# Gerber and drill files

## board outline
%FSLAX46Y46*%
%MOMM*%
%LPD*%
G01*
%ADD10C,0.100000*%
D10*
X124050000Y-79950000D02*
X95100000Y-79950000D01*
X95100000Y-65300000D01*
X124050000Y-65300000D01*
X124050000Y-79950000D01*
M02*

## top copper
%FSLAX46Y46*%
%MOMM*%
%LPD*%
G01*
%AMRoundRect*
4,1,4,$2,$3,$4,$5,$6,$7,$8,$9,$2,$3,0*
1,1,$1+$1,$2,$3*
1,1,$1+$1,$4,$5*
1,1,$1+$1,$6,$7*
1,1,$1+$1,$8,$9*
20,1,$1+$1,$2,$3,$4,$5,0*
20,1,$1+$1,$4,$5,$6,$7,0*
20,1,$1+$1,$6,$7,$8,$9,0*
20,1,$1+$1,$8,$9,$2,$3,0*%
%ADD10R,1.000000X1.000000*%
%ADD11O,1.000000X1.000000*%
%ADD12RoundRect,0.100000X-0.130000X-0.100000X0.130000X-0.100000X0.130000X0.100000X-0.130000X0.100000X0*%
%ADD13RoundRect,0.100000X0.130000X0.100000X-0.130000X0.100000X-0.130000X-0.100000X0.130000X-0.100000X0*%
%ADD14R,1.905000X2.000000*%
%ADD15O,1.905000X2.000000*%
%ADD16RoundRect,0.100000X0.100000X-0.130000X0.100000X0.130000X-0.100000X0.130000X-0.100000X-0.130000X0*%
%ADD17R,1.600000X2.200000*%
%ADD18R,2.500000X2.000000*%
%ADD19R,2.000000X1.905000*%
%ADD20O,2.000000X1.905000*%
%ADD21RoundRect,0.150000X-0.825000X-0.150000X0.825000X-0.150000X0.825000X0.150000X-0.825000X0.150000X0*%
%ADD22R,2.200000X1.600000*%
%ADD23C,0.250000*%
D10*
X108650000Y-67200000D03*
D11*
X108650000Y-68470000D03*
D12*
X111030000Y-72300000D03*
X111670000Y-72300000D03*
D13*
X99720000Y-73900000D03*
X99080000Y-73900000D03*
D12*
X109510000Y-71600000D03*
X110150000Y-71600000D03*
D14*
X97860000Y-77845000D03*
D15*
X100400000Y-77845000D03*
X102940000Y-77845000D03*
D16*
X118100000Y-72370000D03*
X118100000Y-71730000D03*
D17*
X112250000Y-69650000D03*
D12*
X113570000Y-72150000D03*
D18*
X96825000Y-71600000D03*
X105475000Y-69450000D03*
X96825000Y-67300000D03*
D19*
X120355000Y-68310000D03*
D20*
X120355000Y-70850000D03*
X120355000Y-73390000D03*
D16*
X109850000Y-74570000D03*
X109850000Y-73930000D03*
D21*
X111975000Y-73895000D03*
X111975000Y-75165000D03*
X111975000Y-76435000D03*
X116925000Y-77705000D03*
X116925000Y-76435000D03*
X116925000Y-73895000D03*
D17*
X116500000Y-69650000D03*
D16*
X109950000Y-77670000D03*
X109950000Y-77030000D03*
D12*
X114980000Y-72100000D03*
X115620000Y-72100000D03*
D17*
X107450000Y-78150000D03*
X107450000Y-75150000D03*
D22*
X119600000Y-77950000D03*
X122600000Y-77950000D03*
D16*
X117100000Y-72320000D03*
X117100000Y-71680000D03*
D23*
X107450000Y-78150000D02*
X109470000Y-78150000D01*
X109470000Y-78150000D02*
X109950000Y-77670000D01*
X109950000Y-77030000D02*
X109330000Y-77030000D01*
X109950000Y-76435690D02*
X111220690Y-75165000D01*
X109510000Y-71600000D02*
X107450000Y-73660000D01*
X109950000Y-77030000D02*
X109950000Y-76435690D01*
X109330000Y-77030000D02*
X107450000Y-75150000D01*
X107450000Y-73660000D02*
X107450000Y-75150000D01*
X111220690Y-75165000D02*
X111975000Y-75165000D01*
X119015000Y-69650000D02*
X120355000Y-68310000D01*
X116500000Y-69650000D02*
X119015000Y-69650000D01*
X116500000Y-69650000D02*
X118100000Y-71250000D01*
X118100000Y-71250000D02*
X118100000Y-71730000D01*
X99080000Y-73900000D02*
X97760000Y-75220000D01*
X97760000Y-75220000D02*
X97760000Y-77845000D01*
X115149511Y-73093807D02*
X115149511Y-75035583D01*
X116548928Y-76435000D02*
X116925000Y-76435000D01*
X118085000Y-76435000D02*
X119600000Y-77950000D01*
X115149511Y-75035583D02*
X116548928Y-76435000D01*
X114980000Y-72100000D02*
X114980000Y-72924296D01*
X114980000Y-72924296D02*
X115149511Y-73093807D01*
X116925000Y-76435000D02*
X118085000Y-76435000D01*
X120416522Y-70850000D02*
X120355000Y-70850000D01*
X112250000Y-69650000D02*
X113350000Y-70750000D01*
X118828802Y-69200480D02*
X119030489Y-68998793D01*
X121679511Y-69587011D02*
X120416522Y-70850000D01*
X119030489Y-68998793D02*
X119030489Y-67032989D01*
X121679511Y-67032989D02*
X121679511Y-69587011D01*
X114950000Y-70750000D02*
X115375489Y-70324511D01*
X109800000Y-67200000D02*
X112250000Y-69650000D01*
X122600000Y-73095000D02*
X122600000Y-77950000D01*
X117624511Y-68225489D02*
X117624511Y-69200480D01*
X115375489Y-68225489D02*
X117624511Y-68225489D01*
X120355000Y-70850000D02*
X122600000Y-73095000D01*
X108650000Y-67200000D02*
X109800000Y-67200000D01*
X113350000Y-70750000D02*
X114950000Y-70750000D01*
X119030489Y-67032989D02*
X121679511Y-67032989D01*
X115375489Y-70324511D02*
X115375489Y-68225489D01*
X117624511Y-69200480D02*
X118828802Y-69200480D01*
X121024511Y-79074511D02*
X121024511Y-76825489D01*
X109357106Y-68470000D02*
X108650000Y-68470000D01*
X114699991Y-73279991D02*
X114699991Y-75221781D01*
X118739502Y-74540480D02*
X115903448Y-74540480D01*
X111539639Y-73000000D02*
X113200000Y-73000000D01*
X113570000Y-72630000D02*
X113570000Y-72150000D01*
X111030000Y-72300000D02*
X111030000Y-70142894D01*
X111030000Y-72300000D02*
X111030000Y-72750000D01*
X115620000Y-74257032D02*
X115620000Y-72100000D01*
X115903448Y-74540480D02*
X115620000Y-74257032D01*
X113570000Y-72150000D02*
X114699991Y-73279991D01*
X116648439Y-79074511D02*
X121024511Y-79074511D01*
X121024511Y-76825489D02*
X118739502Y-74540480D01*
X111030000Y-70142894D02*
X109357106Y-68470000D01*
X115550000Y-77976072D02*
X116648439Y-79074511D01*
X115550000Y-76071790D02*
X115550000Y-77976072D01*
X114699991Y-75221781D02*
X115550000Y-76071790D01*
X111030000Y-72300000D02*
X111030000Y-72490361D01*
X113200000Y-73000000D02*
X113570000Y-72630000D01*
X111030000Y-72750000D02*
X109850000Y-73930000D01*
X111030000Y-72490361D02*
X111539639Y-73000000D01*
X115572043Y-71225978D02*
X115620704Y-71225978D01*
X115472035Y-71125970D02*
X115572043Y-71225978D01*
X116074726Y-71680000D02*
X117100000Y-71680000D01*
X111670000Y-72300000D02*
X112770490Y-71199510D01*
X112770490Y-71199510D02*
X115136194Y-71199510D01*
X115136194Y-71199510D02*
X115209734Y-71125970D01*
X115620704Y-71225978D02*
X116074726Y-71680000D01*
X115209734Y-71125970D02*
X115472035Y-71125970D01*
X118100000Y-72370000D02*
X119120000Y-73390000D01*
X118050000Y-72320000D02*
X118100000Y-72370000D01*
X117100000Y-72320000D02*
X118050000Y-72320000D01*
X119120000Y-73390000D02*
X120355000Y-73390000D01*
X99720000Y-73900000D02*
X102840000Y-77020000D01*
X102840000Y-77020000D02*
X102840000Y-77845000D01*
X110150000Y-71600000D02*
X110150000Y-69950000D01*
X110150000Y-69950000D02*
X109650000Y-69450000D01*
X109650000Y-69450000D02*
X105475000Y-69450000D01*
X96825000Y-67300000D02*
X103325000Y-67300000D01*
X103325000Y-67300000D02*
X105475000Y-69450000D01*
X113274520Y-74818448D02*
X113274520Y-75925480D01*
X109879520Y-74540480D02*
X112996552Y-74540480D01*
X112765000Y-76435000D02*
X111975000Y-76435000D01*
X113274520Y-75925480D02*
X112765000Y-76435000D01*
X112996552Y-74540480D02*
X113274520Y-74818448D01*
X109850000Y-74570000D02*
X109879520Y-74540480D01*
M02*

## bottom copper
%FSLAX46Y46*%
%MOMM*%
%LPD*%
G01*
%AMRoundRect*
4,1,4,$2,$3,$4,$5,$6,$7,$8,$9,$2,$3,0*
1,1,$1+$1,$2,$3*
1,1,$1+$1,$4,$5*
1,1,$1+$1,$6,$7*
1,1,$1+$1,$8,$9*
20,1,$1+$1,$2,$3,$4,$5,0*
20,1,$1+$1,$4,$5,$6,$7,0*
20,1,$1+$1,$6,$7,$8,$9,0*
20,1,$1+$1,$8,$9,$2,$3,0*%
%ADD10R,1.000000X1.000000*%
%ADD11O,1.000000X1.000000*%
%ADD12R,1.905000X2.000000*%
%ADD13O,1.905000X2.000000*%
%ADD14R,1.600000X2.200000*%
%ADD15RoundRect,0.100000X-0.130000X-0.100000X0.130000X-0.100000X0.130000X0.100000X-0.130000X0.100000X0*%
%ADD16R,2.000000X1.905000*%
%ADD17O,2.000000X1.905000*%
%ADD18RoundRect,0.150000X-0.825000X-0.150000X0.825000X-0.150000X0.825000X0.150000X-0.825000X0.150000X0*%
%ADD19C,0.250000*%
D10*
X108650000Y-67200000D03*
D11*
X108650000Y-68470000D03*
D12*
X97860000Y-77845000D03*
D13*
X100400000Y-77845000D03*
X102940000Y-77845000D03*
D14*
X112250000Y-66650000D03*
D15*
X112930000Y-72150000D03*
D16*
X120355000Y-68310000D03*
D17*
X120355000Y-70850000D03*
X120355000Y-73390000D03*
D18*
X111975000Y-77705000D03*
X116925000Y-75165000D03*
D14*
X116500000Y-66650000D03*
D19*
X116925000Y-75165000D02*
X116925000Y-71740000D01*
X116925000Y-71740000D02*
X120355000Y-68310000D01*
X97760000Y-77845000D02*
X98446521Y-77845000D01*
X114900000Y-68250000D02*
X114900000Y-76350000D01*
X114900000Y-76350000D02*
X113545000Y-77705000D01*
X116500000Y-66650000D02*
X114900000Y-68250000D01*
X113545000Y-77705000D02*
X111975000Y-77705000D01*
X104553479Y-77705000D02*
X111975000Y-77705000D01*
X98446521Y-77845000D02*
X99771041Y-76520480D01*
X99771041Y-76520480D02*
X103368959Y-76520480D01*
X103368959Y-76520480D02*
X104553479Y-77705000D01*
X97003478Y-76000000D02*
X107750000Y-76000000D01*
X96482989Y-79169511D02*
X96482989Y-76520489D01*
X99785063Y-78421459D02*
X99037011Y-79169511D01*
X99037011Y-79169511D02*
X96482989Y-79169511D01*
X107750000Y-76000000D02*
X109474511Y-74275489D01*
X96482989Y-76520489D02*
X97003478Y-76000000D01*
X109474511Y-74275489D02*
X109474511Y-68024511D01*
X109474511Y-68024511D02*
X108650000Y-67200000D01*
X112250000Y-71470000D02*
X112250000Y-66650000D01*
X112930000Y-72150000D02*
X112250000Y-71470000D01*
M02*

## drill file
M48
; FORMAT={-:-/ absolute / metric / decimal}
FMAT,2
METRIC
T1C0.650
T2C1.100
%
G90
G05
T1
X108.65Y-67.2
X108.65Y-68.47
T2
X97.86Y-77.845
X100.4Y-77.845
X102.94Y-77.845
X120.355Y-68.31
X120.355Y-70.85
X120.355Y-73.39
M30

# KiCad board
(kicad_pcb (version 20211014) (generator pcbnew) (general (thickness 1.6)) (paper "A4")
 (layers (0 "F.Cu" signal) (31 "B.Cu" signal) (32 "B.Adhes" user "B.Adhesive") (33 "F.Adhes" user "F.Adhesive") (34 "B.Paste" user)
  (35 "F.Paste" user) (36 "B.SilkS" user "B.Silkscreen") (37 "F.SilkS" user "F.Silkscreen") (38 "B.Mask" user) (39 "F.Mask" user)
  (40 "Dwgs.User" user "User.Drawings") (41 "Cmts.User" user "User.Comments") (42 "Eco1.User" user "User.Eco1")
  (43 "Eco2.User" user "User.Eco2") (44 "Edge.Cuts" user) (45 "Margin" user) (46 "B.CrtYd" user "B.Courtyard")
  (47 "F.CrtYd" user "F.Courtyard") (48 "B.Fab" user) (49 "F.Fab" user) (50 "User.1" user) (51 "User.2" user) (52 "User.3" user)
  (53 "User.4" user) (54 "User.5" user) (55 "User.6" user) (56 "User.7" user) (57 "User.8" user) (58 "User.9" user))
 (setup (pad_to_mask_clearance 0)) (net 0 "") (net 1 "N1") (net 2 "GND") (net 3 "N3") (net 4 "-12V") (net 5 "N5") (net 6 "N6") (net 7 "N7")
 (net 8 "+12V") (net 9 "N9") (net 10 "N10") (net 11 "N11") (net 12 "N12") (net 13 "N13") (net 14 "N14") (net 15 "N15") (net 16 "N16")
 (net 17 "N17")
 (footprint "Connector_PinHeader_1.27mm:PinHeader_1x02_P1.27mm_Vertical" (layer "F.Cu") (at 108.65 67.2)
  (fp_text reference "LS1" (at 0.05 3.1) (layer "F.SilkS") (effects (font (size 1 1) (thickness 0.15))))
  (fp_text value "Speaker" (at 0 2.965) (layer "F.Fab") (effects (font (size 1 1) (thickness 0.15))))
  (pad "1" thru_hole rect (at 0 0) (size 1 1) (drill 0.65) (layers *.Cu *.Mask) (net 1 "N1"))
  (pad "2" thru_hole oval (at 0 1.27) (size 1 1) (drill 0.65) (layers *.Cu *.Mask) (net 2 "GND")))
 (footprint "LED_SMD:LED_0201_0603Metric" (layer "F.Cu") (at 111.35 72.3)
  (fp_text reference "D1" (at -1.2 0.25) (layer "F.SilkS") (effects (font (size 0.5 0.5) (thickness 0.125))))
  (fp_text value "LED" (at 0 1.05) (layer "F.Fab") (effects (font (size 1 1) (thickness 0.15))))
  (pad "" smd roundrect (at 0.345 0) (size 0.318 0.36) (layers "F.Paste") (roundrect_rratio 0.25))
  (pad "" smd roundrect (at -0.345 0) (size 0.318 0.36) (layers "F.Paste") (roundrect_rratio 0.25))
  (pad "1" smd roundrect (at -0.32 0) (size 0.46 0.4) (layers "F.Cu" "F.Mask") (roundrect_rratio 0.25) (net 2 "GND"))
  (pad "2" smd roundrect (at 0.32 0) (size 0.46 0.4) (layers "F.Cu" "F.Mask") (roundrect_rratio 0.25) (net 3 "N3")))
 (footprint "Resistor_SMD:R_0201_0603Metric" (layer "F.Cu") (at 99.4 73.9 180)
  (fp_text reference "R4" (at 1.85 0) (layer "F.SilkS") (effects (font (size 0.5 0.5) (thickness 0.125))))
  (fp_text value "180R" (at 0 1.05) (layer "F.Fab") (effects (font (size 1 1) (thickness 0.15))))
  (pad "" smd roundrect (at 0.345 0 180) (size 0.318 0.36) (layers "F.Paste") (roundrect_rratio 0.25))
  (pad "" smd roundrect (at -0.345 0 180) (size 0.318 0.36) (layers "F.Paste") (roundrect_rratio 0.25))
  (pad "1" smd roundrect (at -0.32 0 180) (size 0.46 0.4) (layers "F.Cu" "F.Mask") (roundrect_rratio 0.25) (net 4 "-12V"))
  (pad "2" smd roundrect (at 0.32 0 180) (size 0.46 0.4) (layers "F.Cu" "F.Mask") (roundrect_rratio 0.25) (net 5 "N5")))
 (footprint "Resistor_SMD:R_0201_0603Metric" (layer "F.Cu") (at 109.83 71.6)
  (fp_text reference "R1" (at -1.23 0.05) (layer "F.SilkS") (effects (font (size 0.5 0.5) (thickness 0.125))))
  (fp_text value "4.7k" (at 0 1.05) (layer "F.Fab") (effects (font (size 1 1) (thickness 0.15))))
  (pad "" smd roundrect (at -0.345 0) (size 0.318 0.36) (layers "F.Paste") (roundrect_rratio 0.25))
  (pad "" smd roundrect (at 0.345 0) (size 0.318 0.36) (layers "F.Paste") (roundrect_rratio 0.25))
  (pad "1" smd roundrect (at -0.32 0) (size 0.46 0.4) (layers "F.Cu" "F.Mask") (roundrect_rratio 0.25) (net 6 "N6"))
  (pad "2" smd roundrect (at 0.32 0) (size 0.46 0.4) (layers "F.Cu" "F.Mask") (roundrect_rratio 0.25) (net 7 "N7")))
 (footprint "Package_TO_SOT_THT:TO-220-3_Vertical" (layer "F.Cu") (at 97.86 77.845)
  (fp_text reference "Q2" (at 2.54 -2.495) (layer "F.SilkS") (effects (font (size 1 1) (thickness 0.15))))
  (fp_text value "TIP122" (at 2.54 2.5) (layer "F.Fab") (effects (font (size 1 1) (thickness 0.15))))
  (pad "1" thru_hole rect (at 0 0) (size 1.905 2) (drill 1.1) (layers *.Cu *.Mask) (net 5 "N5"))
  (pad "2" thru_hole oval (at 2.54 0) (size 1.905 2) (drill 1.1) (layers *.Cu *.Mask) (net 1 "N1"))
  (pad "3" thru_hole oval (at 5.08 0) (size 1.905 2) (drill 1.1) (layers *.Cu *.Mask) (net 4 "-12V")))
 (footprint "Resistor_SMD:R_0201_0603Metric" (layer "F.Cu") (at 118.1 72.05 90)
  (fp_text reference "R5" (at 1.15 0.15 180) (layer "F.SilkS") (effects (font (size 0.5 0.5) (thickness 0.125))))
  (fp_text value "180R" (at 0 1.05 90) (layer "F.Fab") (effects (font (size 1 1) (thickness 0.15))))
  (pad "" smd roundrect (at -0.345 0 90) (size 0.318 0.36) (layers "F.Paste") (roundrect_rratio 0.25))
  (pad "" smd roundrect (at 0.345 0 90) (size 0.318 0.36) (layers "F.Paste") (roundrect_rratio 0.25))
  (pad "1" smd roundrect (at -0.32 0 90) (size 0.46 0.4) (layers "F.Cu" "F.Mask") (roundrect_rratio 0.25) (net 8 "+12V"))
  (pad "2" smd roundrect (at 0.32 0 90) (size 0.46 0.4) (layers "F.Cu" "F.Mask") (roundrect_rratio 0.25) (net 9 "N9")))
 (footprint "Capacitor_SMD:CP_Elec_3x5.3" (layer "F.Cu") (at 112.25 68.15 90)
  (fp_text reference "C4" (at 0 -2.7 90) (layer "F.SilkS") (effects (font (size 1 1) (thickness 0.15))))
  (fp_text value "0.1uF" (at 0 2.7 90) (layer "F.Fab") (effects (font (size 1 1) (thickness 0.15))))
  (pad "1" smd rect (at -1.5 0 90) (size 2.2 1.6) (layers "F.Cu" "F.Paste" "F.Mask") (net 1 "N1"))
  (pad "2" smd rect (at 1.5 0 90) (size 2.2 1.6) (layers "B.Cu" "F.Paste" "F.Mask") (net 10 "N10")))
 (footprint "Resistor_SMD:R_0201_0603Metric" (layer "F.Cu") (at 113.25 72.15)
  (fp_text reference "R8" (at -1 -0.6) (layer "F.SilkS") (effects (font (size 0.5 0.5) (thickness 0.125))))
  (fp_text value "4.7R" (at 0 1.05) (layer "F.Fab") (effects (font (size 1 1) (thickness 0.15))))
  (pad "" smd roundrect (at -0.345 0) (size 0.318 0.36) (layers "F.Paste") (roundrect_rratio 0.25))
  (pad "" smd roundrect (at 0.345 0) (size 0.318 0.36) (layers "F.Paste") (roundrect_rratio 0.25))
  (pad "1" smd roundrect (at -0.32 0) (size 0.46 0.4) (layers "B.Cu" "F.Mask") (roundrect_rratio 0.25) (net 10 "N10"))
  (pad "2" smd roundrect (at 0.32 0) (size 0.46 0.4) (layers "F.Cu" "F.Mask") (roundrect_rratio 0.25) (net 2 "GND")))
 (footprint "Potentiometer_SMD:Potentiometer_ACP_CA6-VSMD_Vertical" (layer "F.Cu") (at 101.15 69.45)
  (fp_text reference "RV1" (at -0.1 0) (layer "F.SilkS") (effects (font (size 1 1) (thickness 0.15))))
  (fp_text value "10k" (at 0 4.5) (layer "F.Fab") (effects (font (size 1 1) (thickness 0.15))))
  (pad "1" smd rect (at -4.325 2.15) (size 2.5 2) (layers "F.Cu" "F.Paste" "F.Mask") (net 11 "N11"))
  (pad "2" smd rect (at 4.325 0) (size 2.5 2) (layers "F.Cu" "F.Paste" "F.Mask") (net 7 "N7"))
  (pad "3" smd rect (at -4.325 -2.15) (size 2.5 2) (layers "F.Cu" "F.Paste" "F.Mask") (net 7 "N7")))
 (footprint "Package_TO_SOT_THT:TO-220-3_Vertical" (layer "F.Cu") (at 120.355 68.31 -90)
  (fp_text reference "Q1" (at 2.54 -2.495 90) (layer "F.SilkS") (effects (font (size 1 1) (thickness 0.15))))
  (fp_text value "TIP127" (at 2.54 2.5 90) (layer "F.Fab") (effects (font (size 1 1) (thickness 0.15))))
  (pad "1" thru_hole rect (at 0 0 270) (size 1.905 2) (drill 1.1) (layers *.Cu *.Mask) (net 9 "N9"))
  (pad "2" thru_hole oval (at 2.54 0 270) (size 1.905 2) (drill 1.1) (layers *.Cu *.Mask) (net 1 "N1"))
  (pad "3" thru_hole oval (at 5.08 0 270) (size 1.905 2) (drill 1.1) (layers *.Cu *.Mask) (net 8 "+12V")))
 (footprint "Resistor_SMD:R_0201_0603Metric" (layer "F.Cu") (at 109.85 74.25 90)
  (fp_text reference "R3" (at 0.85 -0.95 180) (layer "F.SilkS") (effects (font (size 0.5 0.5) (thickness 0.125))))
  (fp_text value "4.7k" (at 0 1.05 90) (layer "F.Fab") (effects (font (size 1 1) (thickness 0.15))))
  (pad "" smd roundrect (at -0.345 0 90) (size 0.318 0.36) (layers "F.Paste") (roundrect_rratio 0.25))
  (pad "" smd roundrect (at 0.345 0 90) (size 0.318 0.36) (layers "F.Paste") (roundrect_rratio 0.25))
  (pad "1" smd roundrect (at -0.32 0 90) (size 0.46 0.4) (layers "F.Cu" "F.Mask") (roundrect_rratio 0.25) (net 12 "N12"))
  (pad "2" smd roundrect (at 0.32 0 90) (size 0.46 0.4) (layers "F.Cu" "F.Mask") (roundrect_rratio 0.25) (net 2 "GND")))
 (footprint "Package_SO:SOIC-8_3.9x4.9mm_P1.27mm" (layer "F.Cu") (at 114.45 75.8)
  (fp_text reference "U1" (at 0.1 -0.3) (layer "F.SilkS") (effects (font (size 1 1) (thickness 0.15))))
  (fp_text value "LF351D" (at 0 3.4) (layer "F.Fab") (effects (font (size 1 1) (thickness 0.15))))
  (pad "1" smd roundrect (at -2.475 -1.905) (size 1.95 0.6) (layers "F.Cu" "F.Paste" "F.Mask") (roundrect_rratio 0.25) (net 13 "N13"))
  (pad "2" smd roundrect (at -2.475 -0.635) (size 1.95 0.6) (layers "F.Cu" "F.Paste" "F.Mask") (roundrect_rratio 0.25) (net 6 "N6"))
  (pad "3" smd roundrect (at -2.475 0.635) (size 1.95 0.6) (layers "F.Cu" "F.Paste" "F.Mask") (roundrect_rratio 0.25) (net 12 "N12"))
  (pad "4" smd roundrect (at -2.475 1.905) (size 1.95 0.6) (layers "B.Cu" "F.Paste" "F.Mask") (roundrect_rratio 0.25) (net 5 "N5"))
  (pad "5" smd roundrect (at 2.475 1.905) (size 1.95 0.6) (layers "F.Cu" "F.Paste" "F.Mask") (roundrect_rratio 0.25) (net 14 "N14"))
  (pad "6" smd roundrect (at 2.475 0.635) (size 1.95 0.6) (layers "F.Cu" "F.Paste" "F.Mask") (roundrect_rratio 0.25) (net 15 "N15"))
  (pad "7" smd roundrect (at 2.475 -0.635) (size 1.95 0.6) (layers "B.Cu" "F.Paste" "F.Mask") (roundrect_rratio 0.25) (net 9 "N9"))
  (pad "8" smd roundrect (at 2.475 -1.905) (size 1.95 0.6) (layers "F.Cu" "F.Paste" "F.Mask") (roundrect_rratio 0.25) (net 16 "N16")))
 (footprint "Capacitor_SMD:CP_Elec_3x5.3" (layer "F.Cu") (at 116.5 68.15 90)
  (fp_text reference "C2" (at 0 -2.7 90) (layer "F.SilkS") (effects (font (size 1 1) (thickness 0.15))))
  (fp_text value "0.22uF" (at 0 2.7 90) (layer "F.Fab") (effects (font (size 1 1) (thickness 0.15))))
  (pad "1" smd rect (at -1.5 0 90) (size 2.2 1.6) (layers "F.Cu" "F.Paste" "F.Mask") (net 9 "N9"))
  (pad "2" smd rect (at 1.5 0 90) (size 2.2 1.6) (layers "B.Cu" "F.Paste" "F.Mask") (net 5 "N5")))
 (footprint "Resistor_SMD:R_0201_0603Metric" (layer "F.Cu") (at 109.95 77.35 90)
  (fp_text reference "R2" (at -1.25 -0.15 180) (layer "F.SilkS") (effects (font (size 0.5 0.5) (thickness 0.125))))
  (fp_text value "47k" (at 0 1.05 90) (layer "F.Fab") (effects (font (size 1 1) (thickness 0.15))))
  (pad "" smd roundrect (at 0.345 0 90) (size 0.318 0.36) (layers "F.Paste") (roundrect_rratio 0.25))
  (pad "" smd roundrect (at -0.345 0 90) (size 0.318 0.36) (layers "F.Paste") (roundrect_rratio 0.25))
  (pad "1" smd roundrect (at -0.32 0 90) (size 0.46 0.4) (layers "F.Cu" "F.Mask") (roundrect_rratio 0.25) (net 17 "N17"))
  (pad "2" smd roundrect (at 0.32 0 90) (size 0.46 0.4) (layers "F.Cu" "F.Mask") (roundrect_rratio 0.25) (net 6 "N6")))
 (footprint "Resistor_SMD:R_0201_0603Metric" (layer "F.Cu") (at 115.3 72.1)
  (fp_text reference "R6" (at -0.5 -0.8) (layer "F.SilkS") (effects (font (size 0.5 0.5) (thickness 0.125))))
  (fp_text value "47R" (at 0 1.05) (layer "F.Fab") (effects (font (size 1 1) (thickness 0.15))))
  (pad "" smd roundrect (at 0.345 0) (size 0.318 0.36) (layers "F.Paste") (roundrect_rratio 0.25))
  (pad "" smd roundrect (at -0.345 0) (size 0.318 0.36) (layers "F.Paste") (roundrect_rratio 0.25))
  (pad "1" smd roundrect (at -0.32 0) (size 0.46 0.4) (layers "F.Cu" "F.Mask") (roundrect_rratio 0.25) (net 15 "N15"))
  (pad "2" smd roundrect (at 0.32 0) (size 0.46 0.4) (layers "F.Cu" "F.Mask") (roundrect_rratio 0.25) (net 2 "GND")))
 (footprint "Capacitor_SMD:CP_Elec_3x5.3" (layer "F.Cu") (at 107.45 76.65 90)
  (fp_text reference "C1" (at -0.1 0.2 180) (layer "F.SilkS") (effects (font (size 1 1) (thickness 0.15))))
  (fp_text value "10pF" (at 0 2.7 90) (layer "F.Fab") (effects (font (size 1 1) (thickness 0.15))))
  (pad "1" smd rect (at -1.5 0 90) (size 2.2 1.6) (layers "F.Cu" "F.Paste" "F.Mask") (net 17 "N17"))
  (pad "2" smd rect (at 1.5 0 90) (size 2.2 1.6) (layers "F.Cu" "F.Paste" "F.Mask") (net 6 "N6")))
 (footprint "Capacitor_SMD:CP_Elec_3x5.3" (layer "F.Cu") (at 121.1 77.95)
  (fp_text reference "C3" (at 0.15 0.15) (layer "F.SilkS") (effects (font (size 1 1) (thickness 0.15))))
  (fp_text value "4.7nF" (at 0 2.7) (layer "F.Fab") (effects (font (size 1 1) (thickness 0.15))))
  (pad "1" smd rect (at -1.5 0) (size 2.2 1.6) (layers "F.Cu" "F.Paste" "F.Mask") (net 15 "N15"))
  (pad "2" smd rect (at 1.5 0) (size 2.2 1.6) (layers "F.Cu" "F.Paste" "F.Mask") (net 1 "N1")))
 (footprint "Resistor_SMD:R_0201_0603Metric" (layer "F.Cu") (at 117.1 72 90)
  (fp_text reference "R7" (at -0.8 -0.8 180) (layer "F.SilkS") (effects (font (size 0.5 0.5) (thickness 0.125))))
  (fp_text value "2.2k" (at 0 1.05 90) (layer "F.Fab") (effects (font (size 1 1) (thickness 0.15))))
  (pad "" smd roundrect (at 0.345 0 90) (size 0.318 0.36) (layers "F.Paste") (roundrect_rratio 0.25))
  (pad "" smd roundrect (at -0.345 0 90) (size 0.318 0.36) (layers "F.Paste") (roundrect_rratio 0.25))
  (pad "1" smd roundrect (at -0.32 0 90) (size 0.46 0.4) (layers "F.Cu" "F.Mask") (roundrect_rratio 0.25) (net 8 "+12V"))
  (pad "2" smd roundrect (at 0.32 0 90) (size 0.46 0.4) (layers "F.Cu" "F.Mask") (roundrect_rratio 0.25) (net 3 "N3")))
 (gr_poly (pts (xy 124.05 79.95) (xy 95.1 79.95) (xy 95.1 65.3) (xy 124.05 65.3)) (layer "Edge.Cuts") (width 0.1) (fill none))
 (segment (start 107.45 78.15) (end 109.47 78.15) (width 0.25) (layer "F.Cu") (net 17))
 (segment (start 109.47 78.15) (end 109.95 77.67) (width 0.25) (layer "F.Cu") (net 17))
 (segment (start 109.95 77.03) (end 109.33 77.03) (width 0.25) (layer "F.Cu") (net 6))
 (segment (start 109.95 76.43569) (end 111.22069 75.165) (width 0.25) (layer "F.Cu") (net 6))
 (segment (start 109.51 71.6) (end 107.45 73.66) (width 0.25) (layer "F.Cu") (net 6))
 (segment (start 109.95 77.03) (end 109.95 76.43569) (width 0.25) (layer "F.Cu") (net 6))
 (segment (start 109.33 77.03) (end 107.45 75.15) (width 0.25) (layer "F.Cu") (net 6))
 (segment (start 107.45 73.66) (end 107.45 75.15) (width 0.25) (layer "F.Cu") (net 6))
 (segment (start 111.22069 75.165) (end 111.975 75.165) (width 0.25) (layer "F.Cu") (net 6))
 (segment (start 119.015 69.65) (end 120.355 68.31) (width 0.25) (layer "F.Cu") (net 9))
 (segment (start 116.5 69.65) (end 119.015 69.65) (width 0.25) (layer "F.Cu") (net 9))
 (segment (start 116.5 69.65) (end 118.1 71.25) (width 0.25) (layer "F.Cu") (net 9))
 (segment (start 118.1 71.25) (end 118.1 71.73) (width 0.25) (layer "F.Cu") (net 9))
 (segment (start 116.925 75.165) (end 116.925 71.74) (width 0.25) (layer "B.Cu") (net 9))
 (segment (start 116.925 71.74) (end 120.355 68.31) (width 0.25) (layer "B.Cu") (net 9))
 (segment (start 99.08 73.9) (end 97.76 75.22) (width 0.25) (layer "F.Cu") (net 5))
 (segment (start 97.76 75.22) (end 97.76 77.845) (width 0.25) (layer "F.Cu") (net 5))
 (segment (start 97.76 77.845) (end 98.446521 77.845) (width 0.25) (layer "B.Cu") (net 5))
 (segment (start 114.9 68.25) (end 114.9 76.35) (width 0.25) (layer "B.Cu") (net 5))
 (segment (start 114.9 76.35) (end 113.545 77.705) (width 0.25) (layer "B.Cu") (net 5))
 (segment (start 116.5 66.65) (end 114.9 68.25) (width 0.25) (layer "B.Cu") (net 5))
 (segment (start 113.545 77.705) (end 111.975 77.705) (width 0.25) (layer "B.Cu") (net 5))
 (segment (start 104.553479 77.705) (end 111.975 77.705) (width 0.25) (layer "B.Cu") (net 5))
 (segment (start 98.446521 77.845) (end 99.771041 76.52048) (width 0.25) (layer "B.Cu") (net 5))
 (segment (start 99.771041 76.52048) (end 103.368959 76.52048) (width 0.25) (layer "B.Cu") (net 5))
 (segment (start 103.368959 76.52048) (end 104.553479 77.705) (width 0.25) (layer "B.Cu") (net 5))
 (segment (start 115.149511 73.093807) (end 115.149511 75.035583) (width 0.25) (layer "F.Cu") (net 15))
 (segment (start 116.548928 76.435) (end 116.925 76.435) (width 0.25) (layer "F.Cu") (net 15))
 (segment (start 118.085 76.435) (end 119.6 77.95) (width 0.25) (layer "F.Cu") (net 15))
 (segment (start 115.149511 75.035583) (end 116.548928 76.435) (width 0.25) (layer "F.Cu") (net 15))
 (segment (start 114.98 72.1) (end 114.98 72.924296) (width 0.25) (layer "F.Cu") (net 15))
 (segment (start 114.98 72.924296) (end 115.149511 73.093807) (width 0.25) (layer "F.Cu") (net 15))
 (segment (start 116.925 76.435) (end 118.085 76.435) (width 0.25) (layer "F.Cu") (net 15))
 (segment (start 120.416522 70.85) (end 120.355 70.85) (width 0.25) (layer "F.Cu") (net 1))
 (segment (start 112.25 69.65) (end 113.35 70.75) (width 0.25) (layer "F.Cu") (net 1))
 (segment (start 118.828802 69.20048) (end 119.030489 68.998793) (width 0.25) (layer "F.Cu") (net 1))
 (segment (start 121.679511 69.587011) (end 120.416522 70.85) (width 0.25) (layer "F.Cu") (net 1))
 (segment (start 119.030489 68.998793) (end 119.030489 67.032989) (width 0.25) (layer "F.Cu") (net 1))
 (segment (start 121.679511 67.032989) (end 121.679511 69.587011) (width 0.25) (layer "F.Cu") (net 1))
 (segment (start 114.95 70.75) (end 115.375489 70.324511) (width 0.25) (layer "F.Cu") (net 1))
 (segment (start 109.8 67.2) (end 112.25 69.65) (width 0.25) (layer "F.Cu") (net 1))
 (segment (start 122.6 73.095) (end 122.6 77.95) (width 0.25) (layer "F.Cu") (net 1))
 (segment (start 117.624511 68.225489) (end 117.624511 69.20048) (width 0.25) (layer "F.Cu") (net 1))
 (segment (start 115.375489 68.225489) (end 117.624511 68.225489) (width 0.25) (layer "F.Cu") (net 1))
 (segment (start 120.355 70.85) (end 122.6 73.095) (width 0.25) (layer "F.Cu") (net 1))
 (segment (start 108.65 67.2) (end 109.8 67.2) (width 0.25) (layer "F.Cu") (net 1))
 (segment (start 113.35 70.75) (end 114.95 70.75) (width 0.25) (layer "F.Cu") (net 1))
 (segment (start 119.030489 67.032989) (end 121.679511 67.032989) (width 0.25) (layer "F.Cu") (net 1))
 (segment (start 115.375489 70.324511) (end 115.375489 68.225489) (width 0.25) (layer "F.Cu") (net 1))
 (segment (start 117.624511 69.20048) (end 118.828802 69.20048) (width 0.25) (layer "F.Cu") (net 1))
 (segment (start 97.003478 76) (end 107.75 76) (width 0.25) (layer "B.Cu") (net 1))
 (segment (start 96.482989 79.169511) (end 96.482989 76.520489) (width 0.25) (layer "B.Cu") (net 1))
 (segment (start 99.785063 78.421459) (end 99.037011 79.169511) (width 0.25) (layer "B.Cu") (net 1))
 (segment (start 99.037011 79.169511) (end 96.482989 79.169511) (width 0.25) (layer "B.Cu") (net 1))
 (segment (start 107.75 76) (end 109.474511 74.275489) (width 0.25) (layer "B.Cu") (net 1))
 (segment (start 96.482989 76.520489) (end 97.003478 76) (width 0.25) (layer "B.Cu") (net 1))
 (segment (start 109.474511 74.275489) (end 109.474511 68.024511) (width 0.25) (layer "B.Cu") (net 1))
 (segment (start 109.474511 68.024511) (end 108.65 67.2) (width 0.25) (layer "B.Cu") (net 1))
 (segment (start 112.25 71.47) (end 112.25 66.65) (width 0.25) (layer "B.Cu") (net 10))
 (segment (start 112.93 72.15) (end 112.25 71.47) (width 0.25) (layer "B.Cu") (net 10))
 (segment (start 121.024511 79.074511) (end 121.024511 76.825489) (width 0.25) (layer "F.Cu") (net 2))
 (segment (start 109.357106 68.47) (end 108.65 68.47) (width 0.25) (layer "F.Cu") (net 2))
 (segment (start 114.699991 73.279991) (end 114.699991 75.221781) (width 0.25) (layer "F.Cu") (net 2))
 (segment (start 118.739502 74.54048) (end 115.903448 74.54048) (width 0.25) (layer "F.Cu") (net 2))
 (segment (start 111.539639 73) (end 113.2 73) (width 0.25) (layer "F.Cu") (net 2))
 (segment (start 113.57 72.63) (end 113.57 72.15) (width 0.25) (layer "F.Cu") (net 2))
 (segment (start 111.03 72.3) (end 111.03 70.142894) (width 0.25) (layer "F.Cu") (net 2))
 (segment (start 111.03 72.3) (end 111.03 72.75) (width 0.25) (layer "F.Cu") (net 2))
 (segment (start 115.62 74.257032) (end 115.62 72.1) (width 0.25) (layer "F.Cu") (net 2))
 (segment (start 115.903448 74.54048) (end 115.62 74.257032) (width 0.25) (layer "F.Cu") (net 2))
 (segment (start 113.57 72.15) (end 114.699991 73.279991) (width 0.25) (layer "F.Cu") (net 2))
 (segment (start 116.648439 79.074511) (end 121.024511 79.074511) (width 0.25) (layer "F.Cu") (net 2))
 (segment (start 121.024511 76.825489) (end 118.739502 74.54048) (width 0.25) (layer "F.Cu") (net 2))
 (segment (start 111.03 70.142894) (end 109.357106 68.47) (width 0.25) (layer "F.Cu") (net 2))
 (segment (start 115.55 77.976072) (end 116.648439 79.074511) (width 0.25) (layer "F.Cu") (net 2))
 (segment (start 115.55 76.07179) (end 115.55 77.976072) (width 0.25) (layer "F.Cu") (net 2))
 (segment (start 114.699991 75.221781) (end 115.55 76.07179) (width 0.25) (layer "F.Cu") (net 2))
 (segment (start 111.03 72.3) (end 111.03 72.490361) (width 0.25) (layer "F.Cu") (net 2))
 (segment (start 113.2 73) (end 113.57 72.63) (width 0.25) (layer "F.Cu") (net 2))
 (segment (start 111.03 72.75) (end 109.85 73.93) (width 0.25) (layer "F.Cu") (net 2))
 (segment (start 111.03 72.490361) (end 111.539639 73) (width 0.25) (layer "F.Cu") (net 2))
 (segment (start 115.572043 71.225978) (end 115.620704 71.225978) (width 0.25) (layer "F.Cu") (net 3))
 (segment (start 115.472035 71.12597) (end 115.572043 71.225978) (width 0.25) (layer "F.Cu") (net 3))
 (segment (start 116.074726 71.68) (end 117.1 71.68) (width 0.25) (layer "F.Cu") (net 3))
 (segment (start 111.67 72.3) (end 112.77049 71.19951) (width 0.25) (layer "F.Cu") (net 3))
 (segment (start 112.77049 71.19951) (end 115.136194 71.19951) (width 0.25) (layer "F.Cu") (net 3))
 (segment (start 115.136194 71.19951) (end 115.209734 71.12597) (width 0.25) (layer "F.Cu") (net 3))
 (segment (start 115.620704 71.225978) (end 116.074726 71.68) (width 0.25) (layer "F.Cu") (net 3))
 (segment (start 115.209734 71.12597) (end 115.472035 71.12597) (width 0.25) (layer "F.Cu") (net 3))
 (segment (start 118.1 72.37) (end 119.12 73.39) (width 0.25) (layer "F.Cu") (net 8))
 (segment (start 118.05 72.32) (end 118.1 72.37) (width 0.25) (layer "F.Cu") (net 8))
 (segment (start 117.1 72.32) (end 118.05 72.32) (width 0.25) (layer "F.Cu") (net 8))
 (segment (start 119.12 73.39) (end 120.355 73.39) (width 0.25) (layer "F.Cu") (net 8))
 (segment (start 99.72 73.9) (end 102.84 77.02) (width 0.25) (layer "F.Cu") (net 4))
 (segment (start 102.84 77.02) (end 102.84 77.845) (width 0.25) (layer "F.Cu") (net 4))
 (segment (start 110.15 71.6) (end 110.15 69.95) (width 0.25) (layer "F.Cu") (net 7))
 (segment (start 110.15 69.95) (end 109.65 69.45) (width 0.25) (layer "F.Cu") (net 7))
 (segment (start 109.65 69.45) (end 105.475 69.45) (width 0.25) (layer "F.Cu") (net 7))
 (segment (start 96.825 67.3) (end 103.325 67.3) (width 0.25) (layer "F.Cu") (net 7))
 (segment (start 103.325 67.3) (end 105.475 69.45) (width 0.25) (layer "F.Cu") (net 7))
 (segment (start 113.27452 74.818448) (end 113.27452 75.92548) (width 0.25) (layer "F.Cu") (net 12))
 (segment (start 109.87952 74.54048) (end 112.996552 74.54048) (width 0.25) (layer "F.Cu") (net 12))
 (segment (start 112.765 76.435) (end 111.975 76.435) (width 0.25) (layer "F.Cu") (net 12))
 (segment (start 113.27452 75.92548) (end 112.765 76.435) (width 0.25) (layer "F.Cu") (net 12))
 (segment (start 112.996552 74.54048) (end 113.27452 74.818448) (width 0.25) (layer "F.Cu") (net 12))
 (segment (start 109.85 74.57) (end 109.87952 74.54048) (width 0.25) (layer "F.Cu") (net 12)))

